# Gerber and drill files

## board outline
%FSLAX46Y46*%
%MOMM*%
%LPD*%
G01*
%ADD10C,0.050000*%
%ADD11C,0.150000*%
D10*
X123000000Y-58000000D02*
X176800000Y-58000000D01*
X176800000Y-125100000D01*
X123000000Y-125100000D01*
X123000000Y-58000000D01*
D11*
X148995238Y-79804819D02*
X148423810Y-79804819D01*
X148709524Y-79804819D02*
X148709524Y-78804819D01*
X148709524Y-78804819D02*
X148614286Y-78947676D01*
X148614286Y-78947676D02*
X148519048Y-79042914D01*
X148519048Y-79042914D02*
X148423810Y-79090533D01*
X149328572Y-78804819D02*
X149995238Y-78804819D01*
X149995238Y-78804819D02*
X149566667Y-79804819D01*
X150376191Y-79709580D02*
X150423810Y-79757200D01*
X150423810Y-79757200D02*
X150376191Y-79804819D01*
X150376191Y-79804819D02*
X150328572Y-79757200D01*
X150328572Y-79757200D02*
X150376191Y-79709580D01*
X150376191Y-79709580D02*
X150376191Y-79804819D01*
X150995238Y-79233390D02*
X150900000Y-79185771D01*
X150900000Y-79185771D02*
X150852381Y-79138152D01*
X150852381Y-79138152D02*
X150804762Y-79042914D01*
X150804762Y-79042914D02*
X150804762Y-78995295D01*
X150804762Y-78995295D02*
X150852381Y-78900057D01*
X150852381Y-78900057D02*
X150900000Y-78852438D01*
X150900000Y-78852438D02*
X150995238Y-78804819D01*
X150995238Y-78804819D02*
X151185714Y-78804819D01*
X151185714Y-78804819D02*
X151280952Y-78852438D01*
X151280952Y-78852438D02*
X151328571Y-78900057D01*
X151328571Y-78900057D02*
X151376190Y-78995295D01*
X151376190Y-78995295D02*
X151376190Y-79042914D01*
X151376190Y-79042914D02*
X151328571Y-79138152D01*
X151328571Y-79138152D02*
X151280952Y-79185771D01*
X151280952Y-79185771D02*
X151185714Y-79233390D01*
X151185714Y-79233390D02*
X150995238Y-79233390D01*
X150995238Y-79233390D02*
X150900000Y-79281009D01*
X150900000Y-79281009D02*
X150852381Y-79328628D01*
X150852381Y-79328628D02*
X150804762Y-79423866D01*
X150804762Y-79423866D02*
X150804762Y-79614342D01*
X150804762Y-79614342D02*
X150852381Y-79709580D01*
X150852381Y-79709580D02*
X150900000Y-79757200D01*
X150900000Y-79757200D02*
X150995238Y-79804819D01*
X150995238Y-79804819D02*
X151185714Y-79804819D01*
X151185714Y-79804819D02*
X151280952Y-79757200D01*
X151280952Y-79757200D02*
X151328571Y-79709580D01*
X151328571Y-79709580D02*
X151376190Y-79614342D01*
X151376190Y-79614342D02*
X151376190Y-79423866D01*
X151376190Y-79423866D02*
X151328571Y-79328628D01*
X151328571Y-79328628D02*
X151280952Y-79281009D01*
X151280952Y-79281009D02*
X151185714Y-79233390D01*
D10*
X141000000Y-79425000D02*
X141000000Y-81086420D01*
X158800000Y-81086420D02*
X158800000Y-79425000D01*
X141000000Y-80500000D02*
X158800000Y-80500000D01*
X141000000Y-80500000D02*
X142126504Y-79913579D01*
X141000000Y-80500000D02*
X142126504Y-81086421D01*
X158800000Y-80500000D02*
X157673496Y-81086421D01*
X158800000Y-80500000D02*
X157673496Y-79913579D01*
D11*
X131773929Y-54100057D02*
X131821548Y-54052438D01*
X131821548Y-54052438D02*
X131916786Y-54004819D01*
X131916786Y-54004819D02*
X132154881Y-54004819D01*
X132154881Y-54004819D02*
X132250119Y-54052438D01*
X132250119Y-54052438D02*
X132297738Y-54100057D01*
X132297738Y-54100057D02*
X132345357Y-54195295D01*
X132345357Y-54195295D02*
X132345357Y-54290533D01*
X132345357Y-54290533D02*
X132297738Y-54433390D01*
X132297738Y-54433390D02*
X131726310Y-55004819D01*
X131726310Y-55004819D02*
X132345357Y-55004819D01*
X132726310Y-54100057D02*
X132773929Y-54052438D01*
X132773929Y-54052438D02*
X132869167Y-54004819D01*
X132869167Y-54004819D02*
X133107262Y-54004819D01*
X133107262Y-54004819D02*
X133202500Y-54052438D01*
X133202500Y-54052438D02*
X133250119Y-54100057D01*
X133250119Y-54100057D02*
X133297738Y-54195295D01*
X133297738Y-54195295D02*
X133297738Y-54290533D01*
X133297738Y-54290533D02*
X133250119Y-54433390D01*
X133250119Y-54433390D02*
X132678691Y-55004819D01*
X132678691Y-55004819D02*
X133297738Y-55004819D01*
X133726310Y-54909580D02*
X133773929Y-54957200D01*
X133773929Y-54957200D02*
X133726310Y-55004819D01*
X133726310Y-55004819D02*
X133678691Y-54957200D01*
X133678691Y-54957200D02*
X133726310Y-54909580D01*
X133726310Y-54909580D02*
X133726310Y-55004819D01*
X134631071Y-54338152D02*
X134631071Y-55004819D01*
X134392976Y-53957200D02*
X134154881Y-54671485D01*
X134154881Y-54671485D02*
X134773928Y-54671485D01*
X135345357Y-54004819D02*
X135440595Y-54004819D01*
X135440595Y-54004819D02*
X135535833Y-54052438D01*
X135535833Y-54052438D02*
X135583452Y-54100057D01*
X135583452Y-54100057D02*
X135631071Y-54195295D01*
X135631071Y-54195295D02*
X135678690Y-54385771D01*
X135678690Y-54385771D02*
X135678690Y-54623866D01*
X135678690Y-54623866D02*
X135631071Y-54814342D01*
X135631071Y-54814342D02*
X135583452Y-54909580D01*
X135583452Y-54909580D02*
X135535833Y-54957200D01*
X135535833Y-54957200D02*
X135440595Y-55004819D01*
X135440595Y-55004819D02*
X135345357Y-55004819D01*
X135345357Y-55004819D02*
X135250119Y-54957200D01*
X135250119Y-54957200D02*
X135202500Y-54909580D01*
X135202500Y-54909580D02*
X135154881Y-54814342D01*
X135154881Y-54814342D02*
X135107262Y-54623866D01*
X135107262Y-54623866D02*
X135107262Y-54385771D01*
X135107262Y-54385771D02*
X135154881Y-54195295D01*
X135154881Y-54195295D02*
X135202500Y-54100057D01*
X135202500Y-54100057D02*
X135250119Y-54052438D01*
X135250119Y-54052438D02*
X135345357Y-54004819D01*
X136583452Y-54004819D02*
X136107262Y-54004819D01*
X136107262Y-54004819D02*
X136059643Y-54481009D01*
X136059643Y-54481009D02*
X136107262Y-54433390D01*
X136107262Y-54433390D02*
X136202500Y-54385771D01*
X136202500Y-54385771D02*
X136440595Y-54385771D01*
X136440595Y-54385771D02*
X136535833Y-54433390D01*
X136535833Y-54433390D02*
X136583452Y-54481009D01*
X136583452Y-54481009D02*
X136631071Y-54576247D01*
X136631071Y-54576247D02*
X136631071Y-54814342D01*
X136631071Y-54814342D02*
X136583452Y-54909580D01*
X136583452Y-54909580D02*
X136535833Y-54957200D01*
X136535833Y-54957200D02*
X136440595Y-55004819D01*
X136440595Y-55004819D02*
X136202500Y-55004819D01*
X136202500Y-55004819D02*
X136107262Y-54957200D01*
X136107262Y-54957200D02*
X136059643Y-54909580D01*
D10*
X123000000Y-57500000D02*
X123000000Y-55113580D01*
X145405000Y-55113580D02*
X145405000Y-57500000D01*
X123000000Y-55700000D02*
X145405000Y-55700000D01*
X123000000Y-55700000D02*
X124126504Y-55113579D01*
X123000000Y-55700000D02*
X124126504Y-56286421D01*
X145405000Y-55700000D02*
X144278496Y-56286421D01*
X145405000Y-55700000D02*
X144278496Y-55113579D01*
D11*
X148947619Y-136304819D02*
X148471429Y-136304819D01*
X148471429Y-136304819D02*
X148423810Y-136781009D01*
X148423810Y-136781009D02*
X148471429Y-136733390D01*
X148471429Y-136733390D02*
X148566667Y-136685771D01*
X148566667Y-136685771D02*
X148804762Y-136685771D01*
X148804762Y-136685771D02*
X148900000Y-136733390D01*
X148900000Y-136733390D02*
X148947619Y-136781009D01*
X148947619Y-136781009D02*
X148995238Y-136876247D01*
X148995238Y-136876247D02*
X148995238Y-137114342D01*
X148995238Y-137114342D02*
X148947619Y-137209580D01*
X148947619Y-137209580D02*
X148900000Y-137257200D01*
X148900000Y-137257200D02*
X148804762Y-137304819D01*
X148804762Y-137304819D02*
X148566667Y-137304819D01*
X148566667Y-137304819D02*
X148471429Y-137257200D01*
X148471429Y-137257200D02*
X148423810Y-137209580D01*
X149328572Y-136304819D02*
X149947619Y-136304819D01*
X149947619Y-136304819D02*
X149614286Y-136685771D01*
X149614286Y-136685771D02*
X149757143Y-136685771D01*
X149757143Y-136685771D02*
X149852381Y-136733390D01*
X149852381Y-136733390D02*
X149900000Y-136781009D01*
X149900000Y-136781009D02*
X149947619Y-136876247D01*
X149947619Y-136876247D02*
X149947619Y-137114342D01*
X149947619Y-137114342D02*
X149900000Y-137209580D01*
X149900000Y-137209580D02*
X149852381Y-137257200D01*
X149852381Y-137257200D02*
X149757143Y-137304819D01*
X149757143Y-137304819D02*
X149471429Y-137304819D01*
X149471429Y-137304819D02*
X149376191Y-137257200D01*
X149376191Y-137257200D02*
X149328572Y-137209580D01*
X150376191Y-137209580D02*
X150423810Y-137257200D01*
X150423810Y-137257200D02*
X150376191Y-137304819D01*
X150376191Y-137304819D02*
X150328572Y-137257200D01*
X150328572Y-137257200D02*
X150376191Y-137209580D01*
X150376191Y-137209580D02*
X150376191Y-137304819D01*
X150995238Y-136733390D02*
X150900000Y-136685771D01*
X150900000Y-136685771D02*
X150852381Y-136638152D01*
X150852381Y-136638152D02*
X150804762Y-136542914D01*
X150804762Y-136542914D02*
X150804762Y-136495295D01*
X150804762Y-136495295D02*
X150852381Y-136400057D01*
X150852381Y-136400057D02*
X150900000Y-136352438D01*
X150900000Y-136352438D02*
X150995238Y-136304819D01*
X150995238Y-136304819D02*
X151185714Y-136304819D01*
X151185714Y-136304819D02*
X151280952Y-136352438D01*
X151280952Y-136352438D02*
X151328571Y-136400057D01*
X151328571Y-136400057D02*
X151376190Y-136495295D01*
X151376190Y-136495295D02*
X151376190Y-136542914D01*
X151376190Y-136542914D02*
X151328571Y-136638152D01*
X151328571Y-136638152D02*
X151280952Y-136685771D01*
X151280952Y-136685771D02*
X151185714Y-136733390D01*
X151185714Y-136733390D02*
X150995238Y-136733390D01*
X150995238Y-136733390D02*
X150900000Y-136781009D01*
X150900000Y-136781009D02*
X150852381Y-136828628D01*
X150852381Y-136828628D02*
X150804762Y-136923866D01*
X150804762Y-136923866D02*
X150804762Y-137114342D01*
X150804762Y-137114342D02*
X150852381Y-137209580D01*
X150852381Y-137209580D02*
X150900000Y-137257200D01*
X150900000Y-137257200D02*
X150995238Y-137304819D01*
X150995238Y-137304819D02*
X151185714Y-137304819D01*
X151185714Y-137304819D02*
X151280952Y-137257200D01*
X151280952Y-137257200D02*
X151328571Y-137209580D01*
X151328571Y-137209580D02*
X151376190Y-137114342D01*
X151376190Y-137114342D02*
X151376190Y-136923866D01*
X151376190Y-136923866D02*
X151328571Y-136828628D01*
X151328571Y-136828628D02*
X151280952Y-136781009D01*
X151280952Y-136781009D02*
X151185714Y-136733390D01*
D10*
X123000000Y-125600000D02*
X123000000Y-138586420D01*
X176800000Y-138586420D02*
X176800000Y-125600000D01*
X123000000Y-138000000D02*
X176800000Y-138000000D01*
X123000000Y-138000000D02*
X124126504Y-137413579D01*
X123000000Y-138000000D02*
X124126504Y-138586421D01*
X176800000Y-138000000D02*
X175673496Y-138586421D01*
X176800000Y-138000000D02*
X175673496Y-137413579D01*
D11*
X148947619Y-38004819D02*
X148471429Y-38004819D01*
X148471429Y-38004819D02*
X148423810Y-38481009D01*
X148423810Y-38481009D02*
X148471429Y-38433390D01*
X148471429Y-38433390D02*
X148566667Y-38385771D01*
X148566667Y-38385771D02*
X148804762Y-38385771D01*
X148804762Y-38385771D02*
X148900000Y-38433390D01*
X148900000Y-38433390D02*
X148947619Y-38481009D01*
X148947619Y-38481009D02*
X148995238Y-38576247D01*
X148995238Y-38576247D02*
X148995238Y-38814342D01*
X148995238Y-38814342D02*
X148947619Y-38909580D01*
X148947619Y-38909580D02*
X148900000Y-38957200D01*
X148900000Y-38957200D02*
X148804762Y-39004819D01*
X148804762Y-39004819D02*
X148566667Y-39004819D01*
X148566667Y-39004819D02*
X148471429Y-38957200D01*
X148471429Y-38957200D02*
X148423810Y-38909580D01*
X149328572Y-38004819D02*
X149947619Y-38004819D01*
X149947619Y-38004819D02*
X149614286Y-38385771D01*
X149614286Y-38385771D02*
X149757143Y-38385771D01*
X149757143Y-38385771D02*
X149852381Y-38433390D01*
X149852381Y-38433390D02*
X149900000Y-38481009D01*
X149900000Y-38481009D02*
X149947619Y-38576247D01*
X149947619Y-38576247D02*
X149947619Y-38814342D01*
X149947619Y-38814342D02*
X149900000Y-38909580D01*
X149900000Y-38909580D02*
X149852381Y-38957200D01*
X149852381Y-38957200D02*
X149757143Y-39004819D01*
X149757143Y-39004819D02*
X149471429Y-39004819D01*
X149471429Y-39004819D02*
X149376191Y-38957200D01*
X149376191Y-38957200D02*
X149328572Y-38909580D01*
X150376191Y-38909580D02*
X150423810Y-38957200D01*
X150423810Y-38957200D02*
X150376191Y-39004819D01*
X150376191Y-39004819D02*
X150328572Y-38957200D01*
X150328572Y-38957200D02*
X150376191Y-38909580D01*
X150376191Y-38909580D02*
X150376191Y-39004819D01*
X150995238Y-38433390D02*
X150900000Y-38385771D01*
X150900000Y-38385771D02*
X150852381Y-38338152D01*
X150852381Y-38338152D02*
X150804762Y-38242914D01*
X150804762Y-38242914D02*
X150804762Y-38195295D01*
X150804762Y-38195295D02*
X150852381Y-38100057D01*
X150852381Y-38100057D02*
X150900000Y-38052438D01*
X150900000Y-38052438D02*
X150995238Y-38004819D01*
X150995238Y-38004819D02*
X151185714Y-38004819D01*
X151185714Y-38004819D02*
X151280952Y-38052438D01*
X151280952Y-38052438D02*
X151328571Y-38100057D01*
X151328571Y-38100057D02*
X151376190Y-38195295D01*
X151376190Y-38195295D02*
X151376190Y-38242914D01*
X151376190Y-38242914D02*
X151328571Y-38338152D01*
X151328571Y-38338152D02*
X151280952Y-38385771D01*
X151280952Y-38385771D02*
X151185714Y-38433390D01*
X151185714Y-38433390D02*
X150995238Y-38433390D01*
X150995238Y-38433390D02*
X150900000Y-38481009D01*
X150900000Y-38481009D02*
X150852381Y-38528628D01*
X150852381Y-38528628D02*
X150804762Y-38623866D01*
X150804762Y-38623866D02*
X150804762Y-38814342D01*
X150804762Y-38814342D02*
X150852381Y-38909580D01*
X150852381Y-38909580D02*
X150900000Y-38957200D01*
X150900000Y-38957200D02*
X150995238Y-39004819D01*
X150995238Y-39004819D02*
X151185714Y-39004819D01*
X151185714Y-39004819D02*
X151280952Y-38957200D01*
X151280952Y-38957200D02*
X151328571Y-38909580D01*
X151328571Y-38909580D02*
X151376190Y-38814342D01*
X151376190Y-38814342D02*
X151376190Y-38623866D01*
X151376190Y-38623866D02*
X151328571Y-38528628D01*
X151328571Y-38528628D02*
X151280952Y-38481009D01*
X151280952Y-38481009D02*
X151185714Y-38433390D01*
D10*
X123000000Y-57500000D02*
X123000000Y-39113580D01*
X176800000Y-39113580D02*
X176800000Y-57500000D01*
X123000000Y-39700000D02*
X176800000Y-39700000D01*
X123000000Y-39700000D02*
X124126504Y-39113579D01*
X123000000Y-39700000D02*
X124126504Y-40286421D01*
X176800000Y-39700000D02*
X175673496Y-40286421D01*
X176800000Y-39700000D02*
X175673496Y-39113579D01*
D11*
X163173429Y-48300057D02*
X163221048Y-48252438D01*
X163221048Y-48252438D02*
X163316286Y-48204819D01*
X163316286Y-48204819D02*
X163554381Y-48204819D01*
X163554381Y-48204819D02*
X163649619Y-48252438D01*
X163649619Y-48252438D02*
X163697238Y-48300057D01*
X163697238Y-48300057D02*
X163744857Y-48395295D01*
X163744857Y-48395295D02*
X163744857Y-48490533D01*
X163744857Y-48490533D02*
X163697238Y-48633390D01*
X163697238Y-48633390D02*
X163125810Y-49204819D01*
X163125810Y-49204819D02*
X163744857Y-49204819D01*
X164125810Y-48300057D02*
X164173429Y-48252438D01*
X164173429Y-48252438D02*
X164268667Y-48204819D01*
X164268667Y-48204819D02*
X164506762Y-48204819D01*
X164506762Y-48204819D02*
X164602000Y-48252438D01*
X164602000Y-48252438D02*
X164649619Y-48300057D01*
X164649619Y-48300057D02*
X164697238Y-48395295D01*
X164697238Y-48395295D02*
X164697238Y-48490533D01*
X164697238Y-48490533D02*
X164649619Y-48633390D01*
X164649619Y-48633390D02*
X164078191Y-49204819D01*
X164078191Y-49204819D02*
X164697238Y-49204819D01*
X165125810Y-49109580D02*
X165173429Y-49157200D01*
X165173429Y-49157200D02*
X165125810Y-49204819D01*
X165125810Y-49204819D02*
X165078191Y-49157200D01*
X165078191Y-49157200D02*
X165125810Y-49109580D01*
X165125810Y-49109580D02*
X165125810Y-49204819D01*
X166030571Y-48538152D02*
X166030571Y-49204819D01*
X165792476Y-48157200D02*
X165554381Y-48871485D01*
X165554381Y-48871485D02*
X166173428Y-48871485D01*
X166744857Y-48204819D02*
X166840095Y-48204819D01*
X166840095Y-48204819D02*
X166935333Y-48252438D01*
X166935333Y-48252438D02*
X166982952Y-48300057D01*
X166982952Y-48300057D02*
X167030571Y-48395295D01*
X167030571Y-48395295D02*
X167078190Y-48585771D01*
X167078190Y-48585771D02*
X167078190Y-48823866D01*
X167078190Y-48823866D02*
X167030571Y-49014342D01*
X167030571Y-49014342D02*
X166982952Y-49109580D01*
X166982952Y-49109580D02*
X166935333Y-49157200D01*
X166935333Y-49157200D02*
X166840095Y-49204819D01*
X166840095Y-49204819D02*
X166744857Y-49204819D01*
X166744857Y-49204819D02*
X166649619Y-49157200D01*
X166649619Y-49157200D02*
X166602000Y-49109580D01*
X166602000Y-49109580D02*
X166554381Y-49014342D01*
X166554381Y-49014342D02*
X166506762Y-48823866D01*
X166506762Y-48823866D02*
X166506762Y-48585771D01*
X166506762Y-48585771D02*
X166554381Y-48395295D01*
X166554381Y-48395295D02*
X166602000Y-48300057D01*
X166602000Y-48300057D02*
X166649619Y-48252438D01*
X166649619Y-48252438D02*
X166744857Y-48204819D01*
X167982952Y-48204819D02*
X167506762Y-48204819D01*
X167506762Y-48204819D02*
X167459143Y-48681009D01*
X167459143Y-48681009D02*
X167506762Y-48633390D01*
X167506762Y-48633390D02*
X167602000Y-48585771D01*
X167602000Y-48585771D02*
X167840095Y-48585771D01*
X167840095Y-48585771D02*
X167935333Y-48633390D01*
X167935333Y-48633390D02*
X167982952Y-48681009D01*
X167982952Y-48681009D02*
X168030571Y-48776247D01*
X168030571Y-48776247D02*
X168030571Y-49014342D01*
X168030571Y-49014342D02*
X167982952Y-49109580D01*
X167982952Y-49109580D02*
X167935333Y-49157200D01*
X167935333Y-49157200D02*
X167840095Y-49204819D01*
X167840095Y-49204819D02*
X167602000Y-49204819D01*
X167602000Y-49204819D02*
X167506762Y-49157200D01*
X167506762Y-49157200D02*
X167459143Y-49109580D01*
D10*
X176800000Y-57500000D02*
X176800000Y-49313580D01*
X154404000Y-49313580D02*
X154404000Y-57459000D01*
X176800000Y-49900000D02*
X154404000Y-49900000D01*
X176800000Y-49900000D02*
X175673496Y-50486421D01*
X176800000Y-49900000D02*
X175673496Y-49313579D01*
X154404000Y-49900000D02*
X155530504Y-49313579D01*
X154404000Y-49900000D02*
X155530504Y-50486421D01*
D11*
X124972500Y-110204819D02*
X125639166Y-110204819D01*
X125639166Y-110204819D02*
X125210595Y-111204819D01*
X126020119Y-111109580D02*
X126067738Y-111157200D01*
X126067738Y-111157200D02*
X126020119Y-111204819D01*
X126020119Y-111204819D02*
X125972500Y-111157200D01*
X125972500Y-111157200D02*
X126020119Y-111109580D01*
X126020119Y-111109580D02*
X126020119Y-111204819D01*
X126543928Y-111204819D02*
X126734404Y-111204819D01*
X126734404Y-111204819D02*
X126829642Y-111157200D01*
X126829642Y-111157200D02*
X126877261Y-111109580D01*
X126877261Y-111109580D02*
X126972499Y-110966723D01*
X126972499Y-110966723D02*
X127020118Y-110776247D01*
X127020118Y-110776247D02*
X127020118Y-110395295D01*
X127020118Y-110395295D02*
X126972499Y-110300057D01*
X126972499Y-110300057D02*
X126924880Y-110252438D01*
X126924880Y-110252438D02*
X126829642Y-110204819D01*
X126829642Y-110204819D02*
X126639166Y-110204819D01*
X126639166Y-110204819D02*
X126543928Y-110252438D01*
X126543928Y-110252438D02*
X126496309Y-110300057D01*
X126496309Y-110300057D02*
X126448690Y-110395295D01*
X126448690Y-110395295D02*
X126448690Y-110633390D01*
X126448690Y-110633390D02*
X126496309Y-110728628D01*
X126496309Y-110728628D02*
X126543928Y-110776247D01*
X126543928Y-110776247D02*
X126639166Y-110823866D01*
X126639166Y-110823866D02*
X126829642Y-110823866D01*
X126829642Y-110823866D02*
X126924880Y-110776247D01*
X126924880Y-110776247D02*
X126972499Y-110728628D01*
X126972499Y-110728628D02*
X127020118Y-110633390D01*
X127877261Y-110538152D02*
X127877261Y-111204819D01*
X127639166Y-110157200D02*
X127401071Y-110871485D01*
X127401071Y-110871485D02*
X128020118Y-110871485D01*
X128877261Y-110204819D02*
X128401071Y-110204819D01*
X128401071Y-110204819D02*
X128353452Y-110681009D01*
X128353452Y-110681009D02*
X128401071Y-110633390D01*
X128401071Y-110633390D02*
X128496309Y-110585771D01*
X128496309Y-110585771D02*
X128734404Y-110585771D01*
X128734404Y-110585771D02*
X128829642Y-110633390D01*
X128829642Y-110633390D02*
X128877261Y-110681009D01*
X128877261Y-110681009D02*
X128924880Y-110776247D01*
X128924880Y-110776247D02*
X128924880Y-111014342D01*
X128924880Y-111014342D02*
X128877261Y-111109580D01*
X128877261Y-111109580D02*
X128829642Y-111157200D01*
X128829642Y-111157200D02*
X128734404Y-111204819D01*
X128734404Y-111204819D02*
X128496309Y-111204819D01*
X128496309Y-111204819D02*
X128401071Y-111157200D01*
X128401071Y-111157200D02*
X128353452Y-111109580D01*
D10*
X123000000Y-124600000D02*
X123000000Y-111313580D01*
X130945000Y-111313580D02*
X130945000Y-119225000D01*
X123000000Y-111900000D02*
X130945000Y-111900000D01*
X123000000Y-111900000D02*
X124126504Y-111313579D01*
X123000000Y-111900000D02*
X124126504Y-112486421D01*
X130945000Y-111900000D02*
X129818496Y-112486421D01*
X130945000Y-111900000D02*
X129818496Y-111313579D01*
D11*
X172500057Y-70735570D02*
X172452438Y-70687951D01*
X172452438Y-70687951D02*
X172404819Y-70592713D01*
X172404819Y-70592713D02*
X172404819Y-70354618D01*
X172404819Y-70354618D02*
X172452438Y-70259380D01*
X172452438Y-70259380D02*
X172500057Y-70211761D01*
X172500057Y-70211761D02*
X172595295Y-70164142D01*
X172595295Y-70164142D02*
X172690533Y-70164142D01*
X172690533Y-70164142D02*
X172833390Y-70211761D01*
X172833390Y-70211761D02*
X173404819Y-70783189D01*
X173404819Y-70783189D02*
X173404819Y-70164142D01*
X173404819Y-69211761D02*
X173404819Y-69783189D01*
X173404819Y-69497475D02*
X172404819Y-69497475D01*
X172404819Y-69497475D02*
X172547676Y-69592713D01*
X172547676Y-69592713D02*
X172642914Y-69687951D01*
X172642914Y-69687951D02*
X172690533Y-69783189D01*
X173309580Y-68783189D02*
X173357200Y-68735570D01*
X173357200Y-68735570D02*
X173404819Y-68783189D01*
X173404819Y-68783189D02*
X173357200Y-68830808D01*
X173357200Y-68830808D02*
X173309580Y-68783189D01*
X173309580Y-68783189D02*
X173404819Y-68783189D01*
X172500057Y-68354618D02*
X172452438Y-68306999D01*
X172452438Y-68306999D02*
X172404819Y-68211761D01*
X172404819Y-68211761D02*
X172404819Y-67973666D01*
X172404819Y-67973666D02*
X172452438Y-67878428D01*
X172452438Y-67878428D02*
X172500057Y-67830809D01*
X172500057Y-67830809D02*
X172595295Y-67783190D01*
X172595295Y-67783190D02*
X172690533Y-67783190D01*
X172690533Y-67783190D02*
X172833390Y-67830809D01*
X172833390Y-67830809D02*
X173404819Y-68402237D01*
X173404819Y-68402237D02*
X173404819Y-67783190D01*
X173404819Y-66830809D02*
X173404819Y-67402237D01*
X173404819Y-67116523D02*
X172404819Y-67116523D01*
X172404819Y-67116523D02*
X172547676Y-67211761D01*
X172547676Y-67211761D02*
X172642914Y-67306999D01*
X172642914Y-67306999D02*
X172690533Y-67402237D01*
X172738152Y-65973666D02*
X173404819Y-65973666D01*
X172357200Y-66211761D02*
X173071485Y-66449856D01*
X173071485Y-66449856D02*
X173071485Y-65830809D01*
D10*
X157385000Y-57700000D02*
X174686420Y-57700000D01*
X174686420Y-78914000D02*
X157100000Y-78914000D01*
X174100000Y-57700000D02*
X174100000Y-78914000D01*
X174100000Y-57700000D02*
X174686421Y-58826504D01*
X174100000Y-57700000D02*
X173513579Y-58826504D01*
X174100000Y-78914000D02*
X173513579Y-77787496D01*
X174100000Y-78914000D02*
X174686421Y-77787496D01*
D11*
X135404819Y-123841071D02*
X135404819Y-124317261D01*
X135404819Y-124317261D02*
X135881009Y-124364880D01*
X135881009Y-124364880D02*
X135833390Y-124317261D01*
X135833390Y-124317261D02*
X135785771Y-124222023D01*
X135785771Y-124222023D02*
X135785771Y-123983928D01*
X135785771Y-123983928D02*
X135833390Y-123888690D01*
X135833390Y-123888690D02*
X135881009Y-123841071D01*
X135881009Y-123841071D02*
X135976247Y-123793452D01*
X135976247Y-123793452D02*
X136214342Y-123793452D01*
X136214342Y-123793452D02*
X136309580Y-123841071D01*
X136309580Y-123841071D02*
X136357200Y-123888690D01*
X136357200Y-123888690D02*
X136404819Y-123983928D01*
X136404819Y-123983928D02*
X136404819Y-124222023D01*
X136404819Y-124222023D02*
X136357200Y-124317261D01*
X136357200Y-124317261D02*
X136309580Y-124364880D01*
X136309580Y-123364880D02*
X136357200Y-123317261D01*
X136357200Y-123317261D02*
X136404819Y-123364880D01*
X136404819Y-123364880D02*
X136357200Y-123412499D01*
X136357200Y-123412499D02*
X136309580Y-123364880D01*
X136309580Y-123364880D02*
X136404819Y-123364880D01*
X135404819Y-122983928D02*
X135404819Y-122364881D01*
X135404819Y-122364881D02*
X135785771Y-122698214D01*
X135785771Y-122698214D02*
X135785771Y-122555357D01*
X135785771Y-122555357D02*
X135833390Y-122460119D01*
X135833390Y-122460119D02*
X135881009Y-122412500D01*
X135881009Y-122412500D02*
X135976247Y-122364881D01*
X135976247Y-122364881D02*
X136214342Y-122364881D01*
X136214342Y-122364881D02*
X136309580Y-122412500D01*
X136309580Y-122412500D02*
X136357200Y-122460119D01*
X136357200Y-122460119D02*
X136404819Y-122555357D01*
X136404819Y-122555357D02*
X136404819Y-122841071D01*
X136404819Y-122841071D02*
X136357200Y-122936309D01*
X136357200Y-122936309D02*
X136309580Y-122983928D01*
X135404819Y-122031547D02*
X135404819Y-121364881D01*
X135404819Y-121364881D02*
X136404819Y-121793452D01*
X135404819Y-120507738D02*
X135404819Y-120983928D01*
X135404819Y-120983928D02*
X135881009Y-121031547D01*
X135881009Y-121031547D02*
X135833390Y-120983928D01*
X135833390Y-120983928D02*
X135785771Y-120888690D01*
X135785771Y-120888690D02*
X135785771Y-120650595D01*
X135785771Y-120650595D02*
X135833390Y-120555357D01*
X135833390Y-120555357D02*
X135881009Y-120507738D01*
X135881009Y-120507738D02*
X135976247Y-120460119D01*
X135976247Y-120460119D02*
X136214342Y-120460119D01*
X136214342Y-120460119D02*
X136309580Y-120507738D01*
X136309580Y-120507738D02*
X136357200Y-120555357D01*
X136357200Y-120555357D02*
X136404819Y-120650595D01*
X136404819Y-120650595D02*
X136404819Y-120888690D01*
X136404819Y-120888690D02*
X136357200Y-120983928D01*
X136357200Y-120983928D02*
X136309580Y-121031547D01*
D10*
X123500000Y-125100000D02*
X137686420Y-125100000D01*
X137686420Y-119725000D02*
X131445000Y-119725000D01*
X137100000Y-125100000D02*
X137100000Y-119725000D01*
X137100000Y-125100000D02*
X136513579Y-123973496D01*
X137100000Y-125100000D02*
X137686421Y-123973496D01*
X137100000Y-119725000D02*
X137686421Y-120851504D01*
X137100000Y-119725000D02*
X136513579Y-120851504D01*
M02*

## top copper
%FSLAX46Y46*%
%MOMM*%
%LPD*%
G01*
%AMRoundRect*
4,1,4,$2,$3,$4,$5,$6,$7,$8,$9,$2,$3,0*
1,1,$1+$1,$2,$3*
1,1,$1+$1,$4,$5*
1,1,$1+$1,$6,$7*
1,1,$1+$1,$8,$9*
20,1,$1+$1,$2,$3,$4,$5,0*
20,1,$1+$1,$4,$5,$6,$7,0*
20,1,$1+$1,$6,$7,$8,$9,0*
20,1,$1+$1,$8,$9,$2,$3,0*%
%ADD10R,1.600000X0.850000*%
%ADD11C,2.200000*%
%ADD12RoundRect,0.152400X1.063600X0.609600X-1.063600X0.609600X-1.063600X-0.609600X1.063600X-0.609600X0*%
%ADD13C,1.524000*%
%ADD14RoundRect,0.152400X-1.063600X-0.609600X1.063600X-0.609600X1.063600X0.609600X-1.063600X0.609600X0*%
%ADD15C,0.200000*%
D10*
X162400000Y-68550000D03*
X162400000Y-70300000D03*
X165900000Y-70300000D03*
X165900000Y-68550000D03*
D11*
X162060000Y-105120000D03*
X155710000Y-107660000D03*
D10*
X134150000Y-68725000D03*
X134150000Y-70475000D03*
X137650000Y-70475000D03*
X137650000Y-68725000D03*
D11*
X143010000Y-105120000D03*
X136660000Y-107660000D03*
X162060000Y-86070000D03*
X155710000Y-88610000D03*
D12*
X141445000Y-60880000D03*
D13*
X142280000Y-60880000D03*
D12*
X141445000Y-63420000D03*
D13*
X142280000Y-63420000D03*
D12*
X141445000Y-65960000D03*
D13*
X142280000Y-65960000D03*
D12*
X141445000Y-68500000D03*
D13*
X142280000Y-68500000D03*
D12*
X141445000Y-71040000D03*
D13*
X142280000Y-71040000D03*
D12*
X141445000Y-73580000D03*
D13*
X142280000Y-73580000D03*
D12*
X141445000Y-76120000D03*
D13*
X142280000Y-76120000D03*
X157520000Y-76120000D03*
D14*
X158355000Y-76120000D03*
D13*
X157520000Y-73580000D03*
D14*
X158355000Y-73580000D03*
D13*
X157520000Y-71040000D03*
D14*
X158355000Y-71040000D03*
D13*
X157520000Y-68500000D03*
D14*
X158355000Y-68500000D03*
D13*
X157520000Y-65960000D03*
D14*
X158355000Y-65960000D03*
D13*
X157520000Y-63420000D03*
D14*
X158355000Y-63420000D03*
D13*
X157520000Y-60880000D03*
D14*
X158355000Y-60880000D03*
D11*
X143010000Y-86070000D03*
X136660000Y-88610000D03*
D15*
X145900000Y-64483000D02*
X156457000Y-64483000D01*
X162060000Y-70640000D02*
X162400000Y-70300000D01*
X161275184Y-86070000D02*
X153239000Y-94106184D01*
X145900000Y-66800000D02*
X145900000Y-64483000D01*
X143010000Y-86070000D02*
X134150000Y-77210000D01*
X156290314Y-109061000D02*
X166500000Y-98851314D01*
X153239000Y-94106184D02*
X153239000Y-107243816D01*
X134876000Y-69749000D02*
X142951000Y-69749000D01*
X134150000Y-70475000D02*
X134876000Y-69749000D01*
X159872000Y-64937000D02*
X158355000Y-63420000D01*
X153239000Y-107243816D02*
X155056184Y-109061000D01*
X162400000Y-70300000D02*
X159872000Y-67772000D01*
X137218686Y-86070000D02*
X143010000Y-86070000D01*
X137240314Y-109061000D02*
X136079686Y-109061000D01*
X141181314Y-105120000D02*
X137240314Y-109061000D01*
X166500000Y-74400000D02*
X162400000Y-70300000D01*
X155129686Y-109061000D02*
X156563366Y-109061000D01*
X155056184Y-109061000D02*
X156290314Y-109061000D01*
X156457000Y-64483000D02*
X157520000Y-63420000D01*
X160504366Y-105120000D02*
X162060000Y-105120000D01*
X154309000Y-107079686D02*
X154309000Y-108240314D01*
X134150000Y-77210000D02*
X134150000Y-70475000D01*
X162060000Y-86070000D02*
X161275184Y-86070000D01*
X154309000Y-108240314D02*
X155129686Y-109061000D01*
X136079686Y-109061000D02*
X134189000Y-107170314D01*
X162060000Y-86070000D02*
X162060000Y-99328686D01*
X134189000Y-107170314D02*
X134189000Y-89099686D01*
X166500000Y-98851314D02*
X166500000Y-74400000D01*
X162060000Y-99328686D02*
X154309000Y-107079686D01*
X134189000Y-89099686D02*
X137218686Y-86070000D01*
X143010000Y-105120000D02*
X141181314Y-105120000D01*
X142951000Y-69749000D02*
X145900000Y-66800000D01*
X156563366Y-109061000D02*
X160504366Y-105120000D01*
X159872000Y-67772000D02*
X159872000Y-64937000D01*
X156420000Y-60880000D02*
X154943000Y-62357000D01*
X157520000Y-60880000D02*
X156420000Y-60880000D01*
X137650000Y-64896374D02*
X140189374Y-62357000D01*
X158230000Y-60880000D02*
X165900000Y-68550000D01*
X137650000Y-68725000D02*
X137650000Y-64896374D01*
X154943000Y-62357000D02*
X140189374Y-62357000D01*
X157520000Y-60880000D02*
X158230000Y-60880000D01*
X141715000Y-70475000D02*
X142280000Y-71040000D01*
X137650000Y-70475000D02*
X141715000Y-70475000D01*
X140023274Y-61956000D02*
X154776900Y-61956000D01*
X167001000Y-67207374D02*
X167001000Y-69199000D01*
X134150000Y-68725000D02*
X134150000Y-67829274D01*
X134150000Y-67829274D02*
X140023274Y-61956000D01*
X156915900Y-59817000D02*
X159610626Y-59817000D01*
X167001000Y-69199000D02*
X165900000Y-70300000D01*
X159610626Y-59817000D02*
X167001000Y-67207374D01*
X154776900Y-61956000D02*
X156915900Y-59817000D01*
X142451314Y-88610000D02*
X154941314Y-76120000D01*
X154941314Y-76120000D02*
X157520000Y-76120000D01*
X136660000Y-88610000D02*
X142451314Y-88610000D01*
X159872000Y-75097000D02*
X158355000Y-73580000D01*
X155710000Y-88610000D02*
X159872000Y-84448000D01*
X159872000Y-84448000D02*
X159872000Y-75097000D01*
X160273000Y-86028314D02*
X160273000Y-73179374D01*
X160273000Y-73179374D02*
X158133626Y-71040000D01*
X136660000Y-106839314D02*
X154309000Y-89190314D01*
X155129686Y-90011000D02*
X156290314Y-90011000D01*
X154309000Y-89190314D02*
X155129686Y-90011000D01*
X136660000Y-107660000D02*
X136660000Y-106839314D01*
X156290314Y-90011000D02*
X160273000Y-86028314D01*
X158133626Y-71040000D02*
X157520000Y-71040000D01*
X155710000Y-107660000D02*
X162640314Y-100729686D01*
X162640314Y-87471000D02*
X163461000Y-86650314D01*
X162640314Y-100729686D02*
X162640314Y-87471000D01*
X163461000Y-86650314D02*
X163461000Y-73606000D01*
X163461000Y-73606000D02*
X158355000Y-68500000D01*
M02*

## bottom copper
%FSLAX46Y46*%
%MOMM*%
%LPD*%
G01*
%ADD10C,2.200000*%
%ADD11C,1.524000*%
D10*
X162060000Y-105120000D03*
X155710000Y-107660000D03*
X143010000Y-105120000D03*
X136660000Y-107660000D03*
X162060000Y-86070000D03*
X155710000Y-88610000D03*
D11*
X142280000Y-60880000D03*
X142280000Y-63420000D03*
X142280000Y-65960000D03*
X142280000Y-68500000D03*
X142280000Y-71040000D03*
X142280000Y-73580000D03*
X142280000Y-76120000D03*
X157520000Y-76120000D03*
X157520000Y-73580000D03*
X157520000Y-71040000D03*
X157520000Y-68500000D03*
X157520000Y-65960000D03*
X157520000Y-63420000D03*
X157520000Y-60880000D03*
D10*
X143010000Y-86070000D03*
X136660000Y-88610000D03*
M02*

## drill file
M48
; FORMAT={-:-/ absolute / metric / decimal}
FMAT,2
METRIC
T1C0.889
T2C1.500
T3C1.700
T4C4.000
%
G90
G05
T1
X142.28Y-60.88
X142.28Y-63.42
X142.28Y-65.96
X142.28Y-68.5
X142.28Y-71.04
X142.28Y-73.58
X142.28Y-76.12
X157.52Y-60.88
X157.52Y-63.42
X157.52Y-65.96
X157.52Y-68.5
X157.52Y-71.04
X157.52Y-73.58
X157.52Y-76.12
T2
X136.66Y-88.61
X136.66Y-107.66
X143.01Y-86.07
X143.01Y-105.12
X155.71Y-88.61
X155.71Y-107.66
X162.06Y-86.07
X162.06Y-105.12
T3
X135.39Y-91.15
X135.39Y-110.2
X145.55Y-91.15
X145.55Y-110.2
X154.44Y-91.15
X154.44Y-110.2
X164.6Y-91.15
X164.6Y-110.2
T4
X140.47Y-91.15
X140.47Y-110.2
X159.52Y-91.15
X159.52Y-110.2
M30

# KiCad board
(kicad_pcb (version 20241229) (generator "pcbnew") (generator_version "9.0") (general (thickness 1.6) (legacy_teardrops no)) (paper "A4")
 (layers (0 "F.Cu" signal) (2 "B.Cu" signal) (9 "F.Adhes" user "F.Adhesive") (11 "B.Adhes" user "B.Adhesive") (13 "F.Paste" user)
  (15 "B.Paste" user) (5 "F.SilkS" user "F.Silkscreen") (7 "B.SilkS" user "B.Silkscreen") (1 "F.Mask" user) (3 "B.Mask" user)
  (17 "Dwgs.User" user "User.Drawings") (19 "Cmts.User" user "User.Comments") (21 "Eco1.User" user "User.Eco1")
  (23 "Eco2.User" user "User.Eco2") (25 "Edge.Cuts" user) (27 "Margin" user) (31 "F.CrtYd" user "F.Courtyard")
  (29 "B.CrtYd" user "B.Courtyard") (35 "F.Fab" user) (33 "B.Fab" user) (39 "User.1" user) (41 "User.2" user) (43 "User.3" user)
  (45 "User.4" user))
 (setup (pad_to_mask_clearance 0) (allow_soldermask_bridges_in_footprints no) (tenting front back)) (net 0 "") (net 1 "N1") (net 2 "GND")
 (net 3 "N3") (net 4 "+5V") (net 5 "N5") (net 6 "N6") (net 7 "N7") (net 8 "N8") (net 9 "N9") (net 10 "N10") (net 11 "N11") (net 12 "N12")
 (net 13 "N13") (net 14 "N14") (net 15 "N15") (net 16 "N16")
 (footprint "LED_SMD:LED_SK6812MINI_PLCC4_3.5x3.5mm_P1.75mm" (layer "F.Cu") (at 164.15 69.425)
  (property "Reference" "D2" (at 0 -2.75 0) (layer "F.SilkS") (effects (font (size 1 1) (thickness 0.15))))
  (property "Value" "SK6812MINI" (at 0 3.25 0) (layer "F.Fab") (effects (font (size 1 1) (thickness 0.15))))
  (pad "1" smd rect (at -1.75 -0.875) (size 1.6 0.85) (layers "F.Cu" "F.Mask" "F.Paste") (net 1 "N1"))
  (pad "2" smd rect (at -1.75 0.875) (size 1.6 0.85) (layers "F.Cu" "F.Mask" "F.Paste") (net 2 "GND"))
  (pad "3" smd rect (at 1.75 0.875) (size 1.6 0.85) (layers "F.Cu" "F.Mask" "F.Paste") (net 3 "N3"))
  (pad "4" smd rect (at 1.75 -0.875) (size 1.6 0.85) (layers "F.Cu" "F.Mask" "F.Paste") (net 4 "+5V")))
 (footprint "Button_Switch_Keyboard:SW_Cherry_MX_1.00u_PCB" (layer "F.Cu") (at 162.06 105.12)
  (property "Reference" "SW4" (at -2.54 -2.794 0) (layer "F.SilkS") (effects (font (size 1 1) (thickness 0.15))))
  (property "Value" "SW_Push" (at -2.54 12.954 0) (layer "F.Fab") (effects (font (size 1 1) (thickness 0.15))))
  (pad "" np_thru_hole circle (at -7.62 5.08) (size 1.7 1.7) (drill 1.7) (layers "*.Cu" "*.Mask"))
  (pad "" np_thru_hole circle (at -2.54 5.08) (size 4 4) (drill 4) (layers "*.Cu" "*.Mask"))
  (pad "" np_thru_hole circle (at 2.54 5.08) (size 1.7 1.7) (drill 1.7) (layers "*.Cu" "*.Mask"))
  (pad "1" thru_hole circle (at 0 0) (size 2.2 2.2) (drill 1.5) (layers "*.Cu" "*.Mask") (remove_unused_layers no) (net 2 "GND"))
  (pad "2" thru_hole circle (at -6.35 2.54) (size 2.2 2.2) (drill 1.5) (layers "*.Cu" "*.Mask") (remove_unused_layers no) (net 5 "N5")))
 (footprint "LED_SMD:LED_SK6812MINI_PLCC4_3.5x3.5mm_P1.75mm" (layer "F.Cu") (at 135.9 69.6)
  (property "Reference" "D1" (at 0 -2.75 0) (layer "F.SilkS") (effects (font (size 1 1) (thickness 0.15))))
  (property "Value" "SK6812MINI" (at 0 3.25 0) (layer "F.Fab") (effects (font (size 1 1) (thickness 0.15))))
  (pad "1" smd rect (at -1.75 -0.875) (size 1.6 0.85) (layers "F.Cu" "F.Mask" "F.Paste") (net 3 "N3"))
  (pad "2" smd rect (at -1.75 0.875) (size 1.6 0.85) (layers "F.Cu" "F.Mask" "F.Paste") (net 2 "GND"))
  (pad "3" smd rect (at 1.75 0.875) (size 1.6 0.85) (layers "F.Cu" "F.Mask" "F.Paste") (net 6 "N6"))
  (pad "4" smd rect (at 1.75 -0.875) (size 1.6 0.85) (layers "F.Cu" "F.Mask" "F.Paste") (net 4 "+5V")))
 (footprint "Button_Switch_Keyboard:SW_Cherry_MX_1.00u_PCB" (layer "F.Cu") (at 143.01 105.12)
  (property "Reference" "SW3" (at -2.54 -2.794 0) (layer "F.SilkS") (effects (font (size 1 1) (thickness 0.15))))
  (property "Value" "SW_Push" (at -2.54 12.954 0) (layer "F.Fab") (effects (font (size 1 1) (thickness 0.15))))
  (pad "" np_thru_hole circle (at -7.62 5.08) (size 1.7 1.7) (drill 1.7) (layers "*.Cu" "*.Mask"))
  (pad "" np_thru_hole circle (at -2.54 5.08) (size 4 4) (drill 4) (layers "*.Cu" "*.Mask"))
  (pad "" np_thru_hole circle (at 2.54 5.08) (size 1.7 1.7) (drill 1.7) (layers "*.Cu" "*.Mask"))
  (pad "1" thru_hole circle (at 0 0) (size 2.2 2.2) (drill 1.5) (layers "*.Cu" "*.Mask") (remove_unused_layers no) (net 2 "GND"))
  (pad "2" thru_hole circle (at -6.35 2.54) (size 2.2 2.2) (drill 1.5) (layers "*.Cu" "*.Mask") (remove_unused_layers no) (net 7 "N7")))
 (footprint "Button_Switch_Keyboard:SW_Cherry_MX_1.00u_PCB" (layer "F.Cu") (at 162.06 86.07)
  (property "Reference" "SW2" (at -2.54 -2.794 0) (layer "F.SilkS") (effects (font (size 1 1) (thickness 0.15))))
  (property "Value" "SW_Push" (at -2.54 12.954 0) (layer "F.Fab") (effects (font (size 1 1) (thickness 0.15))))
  (pad "" np_thru_hole circle (at -7.62 5.08) (size 1.7 1.7) (drill 1.7) (layers "*.Cu" "*.Mask"))
  (pad "" np_thru_hole circle (at -2.54 5.08) (size 4 4) (drill 4) (layers "*.Cu" "*.Mask"))
  (pad "" np_thru_hole circle (at 2.54 5.08) (size 1.7 1.7) (drill 1.7) (layers "*.Cu" "*.Mask"))
  (pad "1" thru_hole circle (at 0 0) (size 2.2 2.2) (drill 1.5) (layers "*.Cu" "*.Mask") (remove_unused_layers no) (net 2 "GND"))
  (pad "2" thru_hole circle (at -6.35 2.54) (size 2.2 2.2) (drill 1.5) (layers "*.Cu" "*.Mask") (remove_unused_layers no) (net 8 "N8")))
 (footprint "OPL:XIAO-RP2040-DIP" (layer "F.Cu") (at 149.9 68.5)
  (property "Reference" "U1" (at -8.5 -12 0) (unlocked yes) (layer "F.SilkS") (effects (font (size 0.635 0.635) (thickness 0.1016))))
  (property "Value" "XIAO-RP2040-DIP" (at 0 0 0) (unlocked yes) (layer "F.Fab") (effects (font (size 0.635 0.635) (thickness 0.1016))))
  (pad "1" smd roundrect (at -8.455 -7.62 180) (size 2.432 1.524) (layers "F.Cu" "F.Mask") (roundrect_rratio 0.1) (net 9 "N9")
   (thermal_bridge_angle 45))
  (pad "1" thru_hole circle (at -7.62 -7.62 180) (size 1.524 1.524) (drill 0.889) (layers "*.Cu" "*.Mask") (remove_unused_layers no)
   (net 9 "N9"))
  (pad "2" smd roundrect (at -8.455 -5.08 180) (size 2.432 1.524) (layers "F.Cu" "F.Mask") (roundrect_rratio 0.1) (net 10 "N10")
   (thermal_bridge_angle 45))
  (pad "2" thru_hole circle (at -7.62 -5.08 180) (size 1.524 1.524) (drill 0.889) (layers "*.Cu" "*.Mask") (remove_unused_layers no)
   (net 10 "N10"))
  (pad "3" smd roundrect (at -8.455 -2.54 180) (size 2.432 1.524) (layers "F.Cu" "F.Mask") (roundrect_rratio 0.1) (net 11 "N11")
   (thermal_bridge_angle 45))
  (pad "3" thru_hole circle (at -7.62 -2.54 180) (size 1.524 1.524) (drill 0.889) (layers "*.Cu" "*.Mask") (remove_unused_layers no)
   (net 11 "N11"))
  (pad "4" smd roundrect (at -8.455 0 180) (size 2.432 1.524) (layers "F.Cu" "F.Mask") (roundrect_rratio 0.1) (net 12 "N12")
   (thermal_bridge_angle 45))
  (pad "4" thru_hole circle (at -7.62 0 180) (size 1.524 1.524) (drill 0.889) (layers "*.Cu" "*.Mask") (remove_unused_layers no)
   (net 12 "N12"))
  (pad "5" smd roundrect (at -8.455 2.54 180) (size 2.432 1.524) (layers "F.Cu" "F.Mask") (roundrect_rratio 0.1) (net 6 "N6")
   (thermal_bridge_angle 45))
  (pad "5" thru_hole circle (at -7.62 2.54 180) (size 1.524 1.524) (drill 0.889) (layers "*.Cu" "*.Mask") (remove_unused_layers no)
   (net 6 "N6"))
  (pad "6" smd roundrect (at -8.455 5.08 180) (size 2.432 1.524) (layers "F.Cu" "F.Mask") (roundrect_rratio 0.1) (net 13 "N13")
   (thermal_bridge_angle 45))
  (pad "6" thru_hole circle (at -7.62 5.08 180) (size 1.524 1.524) (drill 0.889) (layers "*.Cu" "*.Mask") (remove_unused_layers no)
   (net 13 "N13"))
  (pad "7" smd roundrect (at -8.455 7.62 180) (size 2.432 1.524) (layers "F.Cu" "F.Mask") (roundrect_rratio 0.1) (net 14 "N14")
   (thermal_bridge_angle 45))
  (pad "7" thru_hole circle (at -7.62 7.62 180) (size 1.524 1.524) (drill 0.889) (layers "*.Cu" "*.Mask") (remove_unused_layers no)
   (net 14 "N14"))
  (pad "8" thru_hole circle (at 7.62 7.62) (size 1.524 1.524) (drill 0.889) (layers "*.Cu" "*.Mask") (remove_unused_layers no)
   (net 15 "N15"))
  (pad "8" smd roundrect (at 8.455 7.62) (size 2.432 1.524) (layers "F.Cu" "F.Mask") (roundrect_rratio 0.1) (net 15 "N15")
   (thermal_bridge_angle 45))
  (pad "9" thru_hole circle (at 7.62 5.08) (size 1.524 1.524) (drill 0.889) (layers "*.Cu" "*.Mask") (remove_unused_layers no) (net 8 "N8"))
  (pad "9" smd roundrect (at 8.455 5.08) (size 2.432 1.524) (layers "F.Cu" "F.Mask") (roundrect_rratio 0.1) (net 8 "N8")
   (thermal_bridge_angle 45))
  (pad "10" thru_hole circle (at 7.62 2.54) (size 1.524 1.524) (drill 0.889) (layers "*.Cu" "*.Mask") (remove_unused_layers no) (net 7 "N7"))
  (pad "10" smd roundrect (at 8.455 2.54) (size 2.432 1.524) (layers "F.Cu" "F.Mask") (roundrect_rratio 0.1) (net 7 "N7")
   (thermal_bridge_angle 45))
  (pad "11" thru_hole circle (at 7.62 0) (size 1.524 1.524) (drill 0.889) (layers "*.Cu" "*.Mask") (remove_unused_layers no) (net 5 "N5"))
  (pad "11" smd roundrect (at 8.455 0) (size 2.432 1.524) (layers "F.Cu" "F.Mask") (roundrect_rratio 0.1) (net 5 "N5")
   (thermal_bridge_angle 45))
  (pad "12" thru_hole circle (at 7.62 -2.54) (size 1.524 1.524) (drill 0.889) (layers "*.Cu" "*.Mask") (remove_unused_layers no)
   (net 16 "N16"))
  (pad "12" smd roundrect (at 8.455 -2.54) (size 2.432 1.524) (layers "F.Cu" "F.Mask") (roundrect_rratio 0.1) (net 16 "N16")
   (thermal_bridge_angle 45))
  (pad "13" thru_hole circle (at 7.62 -5.08) (size 1.524 1.524) (drill 0.889) (layers "*.Cu" "*.Mask") (remove_unused_layers no)
   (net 2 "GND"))
  (pad "13" smd roundrect (at 8.455 -5.08) (size 2.432 1.524) (layers "F.Cu" "F.Mask") (roundrect_rratio 0.1) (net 2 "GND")
   (thermal_bridge_angle 45))
  (pad "14" thru_hole circle (at 7.62 -7.62) (size 1.524 1.524) (drill 0.889) (layers "*.Cu" "*.Mask") (remove_unused_layers no)
   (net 4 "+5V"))
  (pad "14" smd roundrect (at 8.455 -7.62) (size 2.432 1.524) (layers "F.Cu" "F.Mask") (roundrect_rratio 0.1) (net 4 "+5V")
   (thermal_bridge_angle 45)))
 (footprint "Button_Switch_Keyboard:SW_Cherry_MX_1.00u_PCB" (layer "F.Cu") (at 143.01 86.07)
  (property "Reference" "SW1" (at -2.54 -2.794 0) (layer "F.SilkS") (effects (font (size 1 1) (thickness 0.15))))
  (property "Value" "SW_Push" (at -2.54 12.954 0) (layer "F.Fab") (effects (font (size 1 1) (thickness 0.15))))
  (pad "" np_thru_hole circle (at -7.62 5.08) (size 1.7 1.7) (drill 1.7) (layers "*.Cu" "*.Mask"))
  (pad "" np_thru_hole circle (at -2.54 5.08) (size 4 4) (drill 4) (layers "*.Cu" "*.Mask"))
  (pad "" np_thru_hole circle (at 2.54 5.08) (size 1.7 1.7) (drill 1.7) (layers "*.Cu" "*.Mask"))
  (pad "1" thru_hole circle (at 0 0) (size 2.2 2.2) (drill 1.5) (layers "*.Cu" "*.Mask") (remove_unused_layers no) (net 2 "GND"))
  (pad "2" thru_hole circle (at -6.35 2.54) (size 2.2 2.2) (drill 1.5) (layers "*.Cu" "*.Mask") (remove_unused_layers no) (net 15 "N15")))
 (gr_rect (start 123 58) (end 176.8 125.1) (stroke (width 0.05) (type default)) (fill no) (layer "Edge.Cuts"))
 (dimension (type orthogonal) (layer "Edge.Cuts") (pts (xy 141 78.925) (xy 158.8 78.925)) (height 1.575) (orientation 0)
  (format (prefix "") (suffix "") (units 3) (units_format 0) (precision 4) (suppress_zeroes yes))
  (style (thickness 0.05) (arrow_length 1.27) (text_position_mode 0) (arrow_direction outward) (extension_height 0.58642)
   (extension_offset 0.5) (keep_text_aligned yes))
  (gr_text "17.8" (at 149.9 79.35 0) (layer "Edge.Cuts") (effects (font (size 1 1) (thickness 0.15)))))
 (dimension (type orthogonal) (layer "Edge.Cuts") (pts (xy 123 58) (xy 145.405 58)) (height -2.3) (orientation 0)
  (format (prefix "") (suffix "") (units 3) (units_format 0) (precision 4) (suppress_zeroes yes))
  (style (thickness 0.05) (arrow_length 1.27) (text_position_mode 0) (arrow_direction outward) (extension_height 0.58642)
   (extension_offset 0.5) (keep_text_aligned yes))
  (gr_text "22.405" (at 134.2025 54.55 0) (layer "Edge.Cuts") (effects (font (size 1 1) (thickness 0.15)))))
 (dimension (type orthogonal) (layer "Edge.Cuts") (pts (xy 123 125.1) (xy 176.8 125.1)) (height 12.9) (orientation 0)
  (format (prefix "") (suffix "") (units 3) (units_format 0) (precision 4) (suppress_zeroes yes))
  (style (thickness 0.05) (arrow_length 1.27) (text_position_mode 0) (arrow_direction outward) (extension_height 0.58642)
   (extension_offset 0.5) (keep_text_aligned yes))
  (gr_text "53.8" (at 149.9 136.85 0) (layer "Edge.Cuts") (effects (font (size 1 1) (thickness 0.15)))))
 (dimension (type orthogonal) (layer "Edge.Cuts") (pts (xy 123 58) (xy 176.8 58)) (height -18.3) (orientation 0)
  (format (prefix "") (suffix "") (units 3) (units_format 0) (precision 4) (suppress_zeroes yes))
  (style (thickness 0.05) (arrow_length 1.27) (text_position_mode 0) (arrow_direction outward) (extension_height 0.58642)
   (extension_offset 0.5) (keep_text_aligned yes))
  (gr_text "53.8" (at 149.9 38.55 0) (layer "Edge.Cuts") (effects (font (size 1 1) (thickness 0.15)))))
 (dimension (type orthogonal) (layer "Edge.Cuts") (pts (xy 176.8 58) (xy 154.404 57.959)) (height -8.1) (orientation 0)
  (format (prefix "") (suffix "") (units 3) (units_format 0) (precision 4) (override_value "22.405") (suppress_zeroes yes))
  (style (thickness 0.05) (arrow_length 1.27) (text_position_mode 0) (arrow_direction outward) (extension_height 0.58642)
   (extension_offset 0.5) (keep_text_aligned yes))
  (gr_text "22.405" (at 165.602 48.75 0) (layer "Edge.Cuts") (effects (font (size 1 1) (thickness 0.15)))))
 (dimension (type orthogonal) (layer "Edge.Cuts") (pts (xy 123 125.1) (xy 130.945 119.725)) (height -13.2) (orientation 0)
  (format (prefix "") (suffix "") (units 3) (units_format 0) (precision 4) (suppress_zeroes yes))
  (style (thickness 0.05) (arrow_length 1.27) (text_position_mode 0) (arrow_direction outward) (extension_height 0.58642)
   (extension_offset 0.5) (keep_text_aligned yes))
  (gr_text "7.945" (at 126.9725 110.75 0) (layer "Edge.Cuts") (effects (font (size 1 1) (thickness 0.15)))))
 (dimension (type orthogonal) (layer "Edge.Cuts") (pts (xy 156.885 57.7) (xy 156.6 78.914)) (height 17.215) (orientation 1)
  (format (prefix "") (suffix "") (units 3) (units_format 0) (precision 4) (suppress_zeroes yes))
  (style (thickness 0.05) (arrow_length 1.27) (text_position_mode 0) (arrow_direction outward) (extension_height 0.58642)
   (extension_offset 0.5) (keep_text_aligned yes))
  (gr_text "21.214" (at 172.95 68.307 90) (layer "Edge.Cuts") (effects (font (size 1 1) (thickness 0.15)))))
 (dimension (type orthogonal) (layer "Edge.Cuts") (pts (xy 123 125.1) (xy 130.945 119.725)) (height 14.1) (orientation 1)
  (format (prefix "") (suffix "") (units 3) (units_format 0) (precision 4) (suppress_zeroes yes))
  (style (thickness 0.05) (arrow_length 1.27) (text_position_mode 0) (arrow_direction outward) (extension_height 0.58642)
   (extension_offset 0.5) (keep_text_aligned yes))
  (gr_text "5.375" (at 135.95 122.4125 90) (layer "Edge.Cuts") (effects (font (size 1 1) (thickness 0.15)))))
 (segment (start 145.9 64.483) (end 156.457 64.483) (width 0.2) (layer "F.Cu") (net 2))
 (segment (start 162.06 70.64) (end 162.4 70.3) (width 0.2) (layer "F.Cu") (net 2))
 (segment (start 161.275184 86.07) (end 153.239 94.106184) (width 0.2) (layer "F.Cu") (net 2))
 (segment (start 145.9 66.8) (end 145.9 64.483) (width 0.2) (layer "F.Cu") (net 2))
 (segment (start 143.01 86.07) (end 134.15 77.21) (width 0.2) (layer "F.Cu") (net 2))
 (segment (start 156.290314 109.061) (end 166.5 98.851314) (width 0.2) (layer "F.Cu") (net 2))
 (segment (start 153.239 94.106184) (end 153.239 107.243816) (width 0.2) (layer "F.Cu") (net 2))
 (segment (start 134.876 69.749) (end 142.951 69.749) (width 0.2) (layer "F.Cu") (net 2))
 (segment (start 134.15 70.475) (end 134.876 69.749) (width 0.2) (layer "F.Cu") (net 2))
 (segment (start 159.872 64.937) (end 158.355 63.42) (width 0.2) (layer "F.Cu") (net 2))
 (segment (start 153.239 107.243816) (end 155.056184 109.061) (width 0.2) (layer "F.Cu") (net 2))
 (segment (start 162.4 70.3) (end 159.872 67.772) (width 0.2) (layer "F.Cu") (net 2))
 (segment (start 137.218686 86.07) (end 143.01 86.07) (width 0.2) (layer "F.Cu") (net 2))
 (segment (start 137.240314 109.061) (end 136.079686 109.061) (width 0.2) (layer "F.Cu") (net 2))
 (segment (start 141.181314 105.12) (end 137.240314 109.061) (width 0.2) (layer "F.Cu") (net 2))
 (segment (start 166.5 74.4) (end 162.4 70.3) (width 0.2) (layer "F.Cu") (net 2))
 (segment (start 155.129686 109.061) (end 156.563366 109.061) (width 0.2) (layer "F.Cu") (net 2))
 (segment (start 155.056184 109.061) (end 156.290314 109.061) (width 0.2) (layer "F.Cu") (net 2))
 (segment (start 156.457 64.483) (end 157.52 63.42) (width 0.2) (layer "F.Cu") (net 2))
 (segment (start 160.504366 105.12) (end 162.06 105.12) (width 0.2) (layer "F.Cu") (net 2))
 (segment (start 154.309 107.079686) (end 154.309 108.240314) (width 0.2) (layer "F.Cu") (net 2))
 (segment (start 134.15 77.21) (end 134.15 70.475) (width 0.2) (layer "F.Cu") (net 2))
 (segment (start 162.06 86.07) (end 161.275184 86.07) (width 0.2) (layer "F.Cu") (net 2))
 (segment (start 154.309 108.240314) (end 155.129686 109.061) (width 0.2) (layer "F.Cu") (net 2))
 (segment (start 136.079686 109.061) (end 134.189 107.170314) (width 0.2) (layer "F.Cu") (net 2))
 (segment (start 162.06 86.07) (end 162.06 99.328686) (width 0.2) (layer "F.Cu") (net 2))
 (segment (start 134.189 107.170314) (end 134.189 89.099686) (width 0.2) (layer "F.Cu") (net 2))
 (segment (start 166.5 98.851314) (end 166.5 74.4) (width 0.2) (layer "F.Cu") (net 2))
 (segment (start 162.06 99.328686) (end 154.309 107.079686) (width 0.2) (layer "F.Cu") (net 2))
 (segment (start 134.189 89.099686) (end 137.218686 86.07) (width 0.2) (layer "F.Cu") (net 2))
 (segment (start 143.01 105.12) (end 141.181314 105.12) (width 0.2) (layer "F.Cu") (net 2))
 (segment (start 142.951 69.749) (end 145.9 66.8) (width 0.2) (layer "F.Cu") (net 2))
 (segment (start 156.563366 109.061) (end 160.504366 105.12) (width 0.2) (layer "F.Cu") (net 2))
 (segment (start 159.872 67.772) (end 159.872 64.937) (width 0.2) (layer "F.Cu") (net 2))
 (segment (start 156.42 60.88) (end 154.943 62.357) (width 0.2) (layer "F.Cu") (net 4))
 (segment (start 157.52 60.88) (end 156.42 60.88) (width 0.2) (layer "F.Cu") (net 4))
 (segment (start 137.65 64.896374) (end 140.189374 62.357) (width 0.2) (layer "F.Cu") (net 4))
 (segment (start 158.23 60.88) (end 165.9 68.55) (width 0.2) (layer "F.Cu") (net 4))
 (segment (start 137.65 68.725) (end 137.65 64.896374) (width 0.2) (layer "F.Cu") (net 4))
 (segment (start 154.943 62.357) (end 140.189374 62.357) (width 0.2) (layer "F.Cu") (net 4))
 (segment (start 157.52 60.88) (end 158.23 60.88) (width 0.2) (layer "F.Cu") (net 4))
 (segment (start 141.715 70.475) (end 142.28 71.04) (width 0.2) (layer "F.Cu") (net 6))
 (segment (start 137.65 70.475) (end 141.715 70.475) (width 0.2) (layer "F.Cu") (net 6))
 (segment (start 140.023274 61.956) (end 154.7769 61.956) (width 0.2) (layer "F.Cu") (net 3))
 (segment (start 167.001 67.207374) (end 167.001 69.199) (width 0.2) (layer "F.Cu") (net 3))
 (segment (start 134.15 68.725) (end 134.15 67.829274) (width 0.2) (layer "F.Cu") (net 3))
 (segment (start 134.15 67.829274) (end 140.023274 61.956) (width 0.2) (layer "F.Cu") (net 3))
 (segment (start 156.9159 59.817) (end 159.610626 59.817) (width 0.2) (layer "F.Cu") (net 3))
 (segment (start 167.001 69.199) (end 165.9 70.3) (width 0.2) (layer "F.Cu") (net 3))
 (segment (start 159.610626 59.817) (end 167.001 67.207374) (width 0.2) (layer "F.Cu") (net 3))
 (segment (start 154.7769 61.956) (end 156.9159 59.817) (width 0.2) (layer "F.Cu") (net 3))
 (segment (start 142.451314 88.61) (end 154.941314 76.12) (width 0.2) (layer "F.Cu") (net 15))
 (segment (start 154.941314 76.12) (end 157.52 76.12) (width 0.2) (layer "F.Cu") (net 15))
 (segment (start 136.66 88.61) (end 142.451314 88.61) (width 0.2) (layer "F.Cu") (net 15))
 (segment (start 159.872 75.097) (end 158.355 73.58) (width 0.2) (layer "F.Cu") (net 8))
 (segment (start 155.71 88.61) (end 159.872 84.448) (width 0.2) (layer "F.Cu") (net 8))
 (segment (start 159.872 84.448) (end 159.872 75.097) (width 0.2) (layer "F.Cu") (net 8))
 (segment (start 160.273 86.028314) (end 160.273 73.179374) (width 0.2) (layer "F.Cu") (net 7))
 (segment (start 160.273 73.179374) (end 158.133626 71.04) (width 0.2) (layer "F.Cu") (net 7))
 (segment (start 136.66 106.839314) (end 154.309 89.190314) (width 0.2) (layer "F.Cu") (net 7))
 (segment (start 155.129686 90.011) (end 156.290314 90.011) (width 0.2) (layer "F.Cu") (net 7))
 (segment (start 154.309 89.190314) (end 155.129686 90.011) (width 0.2) (layer "F.Cu") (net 7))
 (segment (start 136.66 107.66) (end 136.66 106.839314) (width 0.2) (layer "F.Cu") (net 7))
 (segment (start 156.290314 90.011) (end 160.273 86.028314) (width 0.2) (layer "F.Cu") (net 7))
 (segment (start 158.133626 71.04) (end 157.52 71.04) (width 0.2) (layer "F.Cu") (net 7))
 (segment (start 155.71 107.66) (end 162.640314 100.729686) (width 0.2) (layer "F.Cu") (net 5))
 (segment (start 162.640314 87.471) (end 163.461 86.650314) (width 0.2) (layer "F.Cu") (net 5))
 (segment (start 162.640314 100.729686) (end 162.640314 87.471) (width 0.2) (layer "F.Cu") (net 5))
 (segment (start 163.461 86.650314) (end 163.461 73.606) (width 0.2) (layer "F.Cu") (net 5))
 (segment (start 163.461 73.606) (end 158.355 68.5) (width 0.2) (layer "F.Cu") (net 5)))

